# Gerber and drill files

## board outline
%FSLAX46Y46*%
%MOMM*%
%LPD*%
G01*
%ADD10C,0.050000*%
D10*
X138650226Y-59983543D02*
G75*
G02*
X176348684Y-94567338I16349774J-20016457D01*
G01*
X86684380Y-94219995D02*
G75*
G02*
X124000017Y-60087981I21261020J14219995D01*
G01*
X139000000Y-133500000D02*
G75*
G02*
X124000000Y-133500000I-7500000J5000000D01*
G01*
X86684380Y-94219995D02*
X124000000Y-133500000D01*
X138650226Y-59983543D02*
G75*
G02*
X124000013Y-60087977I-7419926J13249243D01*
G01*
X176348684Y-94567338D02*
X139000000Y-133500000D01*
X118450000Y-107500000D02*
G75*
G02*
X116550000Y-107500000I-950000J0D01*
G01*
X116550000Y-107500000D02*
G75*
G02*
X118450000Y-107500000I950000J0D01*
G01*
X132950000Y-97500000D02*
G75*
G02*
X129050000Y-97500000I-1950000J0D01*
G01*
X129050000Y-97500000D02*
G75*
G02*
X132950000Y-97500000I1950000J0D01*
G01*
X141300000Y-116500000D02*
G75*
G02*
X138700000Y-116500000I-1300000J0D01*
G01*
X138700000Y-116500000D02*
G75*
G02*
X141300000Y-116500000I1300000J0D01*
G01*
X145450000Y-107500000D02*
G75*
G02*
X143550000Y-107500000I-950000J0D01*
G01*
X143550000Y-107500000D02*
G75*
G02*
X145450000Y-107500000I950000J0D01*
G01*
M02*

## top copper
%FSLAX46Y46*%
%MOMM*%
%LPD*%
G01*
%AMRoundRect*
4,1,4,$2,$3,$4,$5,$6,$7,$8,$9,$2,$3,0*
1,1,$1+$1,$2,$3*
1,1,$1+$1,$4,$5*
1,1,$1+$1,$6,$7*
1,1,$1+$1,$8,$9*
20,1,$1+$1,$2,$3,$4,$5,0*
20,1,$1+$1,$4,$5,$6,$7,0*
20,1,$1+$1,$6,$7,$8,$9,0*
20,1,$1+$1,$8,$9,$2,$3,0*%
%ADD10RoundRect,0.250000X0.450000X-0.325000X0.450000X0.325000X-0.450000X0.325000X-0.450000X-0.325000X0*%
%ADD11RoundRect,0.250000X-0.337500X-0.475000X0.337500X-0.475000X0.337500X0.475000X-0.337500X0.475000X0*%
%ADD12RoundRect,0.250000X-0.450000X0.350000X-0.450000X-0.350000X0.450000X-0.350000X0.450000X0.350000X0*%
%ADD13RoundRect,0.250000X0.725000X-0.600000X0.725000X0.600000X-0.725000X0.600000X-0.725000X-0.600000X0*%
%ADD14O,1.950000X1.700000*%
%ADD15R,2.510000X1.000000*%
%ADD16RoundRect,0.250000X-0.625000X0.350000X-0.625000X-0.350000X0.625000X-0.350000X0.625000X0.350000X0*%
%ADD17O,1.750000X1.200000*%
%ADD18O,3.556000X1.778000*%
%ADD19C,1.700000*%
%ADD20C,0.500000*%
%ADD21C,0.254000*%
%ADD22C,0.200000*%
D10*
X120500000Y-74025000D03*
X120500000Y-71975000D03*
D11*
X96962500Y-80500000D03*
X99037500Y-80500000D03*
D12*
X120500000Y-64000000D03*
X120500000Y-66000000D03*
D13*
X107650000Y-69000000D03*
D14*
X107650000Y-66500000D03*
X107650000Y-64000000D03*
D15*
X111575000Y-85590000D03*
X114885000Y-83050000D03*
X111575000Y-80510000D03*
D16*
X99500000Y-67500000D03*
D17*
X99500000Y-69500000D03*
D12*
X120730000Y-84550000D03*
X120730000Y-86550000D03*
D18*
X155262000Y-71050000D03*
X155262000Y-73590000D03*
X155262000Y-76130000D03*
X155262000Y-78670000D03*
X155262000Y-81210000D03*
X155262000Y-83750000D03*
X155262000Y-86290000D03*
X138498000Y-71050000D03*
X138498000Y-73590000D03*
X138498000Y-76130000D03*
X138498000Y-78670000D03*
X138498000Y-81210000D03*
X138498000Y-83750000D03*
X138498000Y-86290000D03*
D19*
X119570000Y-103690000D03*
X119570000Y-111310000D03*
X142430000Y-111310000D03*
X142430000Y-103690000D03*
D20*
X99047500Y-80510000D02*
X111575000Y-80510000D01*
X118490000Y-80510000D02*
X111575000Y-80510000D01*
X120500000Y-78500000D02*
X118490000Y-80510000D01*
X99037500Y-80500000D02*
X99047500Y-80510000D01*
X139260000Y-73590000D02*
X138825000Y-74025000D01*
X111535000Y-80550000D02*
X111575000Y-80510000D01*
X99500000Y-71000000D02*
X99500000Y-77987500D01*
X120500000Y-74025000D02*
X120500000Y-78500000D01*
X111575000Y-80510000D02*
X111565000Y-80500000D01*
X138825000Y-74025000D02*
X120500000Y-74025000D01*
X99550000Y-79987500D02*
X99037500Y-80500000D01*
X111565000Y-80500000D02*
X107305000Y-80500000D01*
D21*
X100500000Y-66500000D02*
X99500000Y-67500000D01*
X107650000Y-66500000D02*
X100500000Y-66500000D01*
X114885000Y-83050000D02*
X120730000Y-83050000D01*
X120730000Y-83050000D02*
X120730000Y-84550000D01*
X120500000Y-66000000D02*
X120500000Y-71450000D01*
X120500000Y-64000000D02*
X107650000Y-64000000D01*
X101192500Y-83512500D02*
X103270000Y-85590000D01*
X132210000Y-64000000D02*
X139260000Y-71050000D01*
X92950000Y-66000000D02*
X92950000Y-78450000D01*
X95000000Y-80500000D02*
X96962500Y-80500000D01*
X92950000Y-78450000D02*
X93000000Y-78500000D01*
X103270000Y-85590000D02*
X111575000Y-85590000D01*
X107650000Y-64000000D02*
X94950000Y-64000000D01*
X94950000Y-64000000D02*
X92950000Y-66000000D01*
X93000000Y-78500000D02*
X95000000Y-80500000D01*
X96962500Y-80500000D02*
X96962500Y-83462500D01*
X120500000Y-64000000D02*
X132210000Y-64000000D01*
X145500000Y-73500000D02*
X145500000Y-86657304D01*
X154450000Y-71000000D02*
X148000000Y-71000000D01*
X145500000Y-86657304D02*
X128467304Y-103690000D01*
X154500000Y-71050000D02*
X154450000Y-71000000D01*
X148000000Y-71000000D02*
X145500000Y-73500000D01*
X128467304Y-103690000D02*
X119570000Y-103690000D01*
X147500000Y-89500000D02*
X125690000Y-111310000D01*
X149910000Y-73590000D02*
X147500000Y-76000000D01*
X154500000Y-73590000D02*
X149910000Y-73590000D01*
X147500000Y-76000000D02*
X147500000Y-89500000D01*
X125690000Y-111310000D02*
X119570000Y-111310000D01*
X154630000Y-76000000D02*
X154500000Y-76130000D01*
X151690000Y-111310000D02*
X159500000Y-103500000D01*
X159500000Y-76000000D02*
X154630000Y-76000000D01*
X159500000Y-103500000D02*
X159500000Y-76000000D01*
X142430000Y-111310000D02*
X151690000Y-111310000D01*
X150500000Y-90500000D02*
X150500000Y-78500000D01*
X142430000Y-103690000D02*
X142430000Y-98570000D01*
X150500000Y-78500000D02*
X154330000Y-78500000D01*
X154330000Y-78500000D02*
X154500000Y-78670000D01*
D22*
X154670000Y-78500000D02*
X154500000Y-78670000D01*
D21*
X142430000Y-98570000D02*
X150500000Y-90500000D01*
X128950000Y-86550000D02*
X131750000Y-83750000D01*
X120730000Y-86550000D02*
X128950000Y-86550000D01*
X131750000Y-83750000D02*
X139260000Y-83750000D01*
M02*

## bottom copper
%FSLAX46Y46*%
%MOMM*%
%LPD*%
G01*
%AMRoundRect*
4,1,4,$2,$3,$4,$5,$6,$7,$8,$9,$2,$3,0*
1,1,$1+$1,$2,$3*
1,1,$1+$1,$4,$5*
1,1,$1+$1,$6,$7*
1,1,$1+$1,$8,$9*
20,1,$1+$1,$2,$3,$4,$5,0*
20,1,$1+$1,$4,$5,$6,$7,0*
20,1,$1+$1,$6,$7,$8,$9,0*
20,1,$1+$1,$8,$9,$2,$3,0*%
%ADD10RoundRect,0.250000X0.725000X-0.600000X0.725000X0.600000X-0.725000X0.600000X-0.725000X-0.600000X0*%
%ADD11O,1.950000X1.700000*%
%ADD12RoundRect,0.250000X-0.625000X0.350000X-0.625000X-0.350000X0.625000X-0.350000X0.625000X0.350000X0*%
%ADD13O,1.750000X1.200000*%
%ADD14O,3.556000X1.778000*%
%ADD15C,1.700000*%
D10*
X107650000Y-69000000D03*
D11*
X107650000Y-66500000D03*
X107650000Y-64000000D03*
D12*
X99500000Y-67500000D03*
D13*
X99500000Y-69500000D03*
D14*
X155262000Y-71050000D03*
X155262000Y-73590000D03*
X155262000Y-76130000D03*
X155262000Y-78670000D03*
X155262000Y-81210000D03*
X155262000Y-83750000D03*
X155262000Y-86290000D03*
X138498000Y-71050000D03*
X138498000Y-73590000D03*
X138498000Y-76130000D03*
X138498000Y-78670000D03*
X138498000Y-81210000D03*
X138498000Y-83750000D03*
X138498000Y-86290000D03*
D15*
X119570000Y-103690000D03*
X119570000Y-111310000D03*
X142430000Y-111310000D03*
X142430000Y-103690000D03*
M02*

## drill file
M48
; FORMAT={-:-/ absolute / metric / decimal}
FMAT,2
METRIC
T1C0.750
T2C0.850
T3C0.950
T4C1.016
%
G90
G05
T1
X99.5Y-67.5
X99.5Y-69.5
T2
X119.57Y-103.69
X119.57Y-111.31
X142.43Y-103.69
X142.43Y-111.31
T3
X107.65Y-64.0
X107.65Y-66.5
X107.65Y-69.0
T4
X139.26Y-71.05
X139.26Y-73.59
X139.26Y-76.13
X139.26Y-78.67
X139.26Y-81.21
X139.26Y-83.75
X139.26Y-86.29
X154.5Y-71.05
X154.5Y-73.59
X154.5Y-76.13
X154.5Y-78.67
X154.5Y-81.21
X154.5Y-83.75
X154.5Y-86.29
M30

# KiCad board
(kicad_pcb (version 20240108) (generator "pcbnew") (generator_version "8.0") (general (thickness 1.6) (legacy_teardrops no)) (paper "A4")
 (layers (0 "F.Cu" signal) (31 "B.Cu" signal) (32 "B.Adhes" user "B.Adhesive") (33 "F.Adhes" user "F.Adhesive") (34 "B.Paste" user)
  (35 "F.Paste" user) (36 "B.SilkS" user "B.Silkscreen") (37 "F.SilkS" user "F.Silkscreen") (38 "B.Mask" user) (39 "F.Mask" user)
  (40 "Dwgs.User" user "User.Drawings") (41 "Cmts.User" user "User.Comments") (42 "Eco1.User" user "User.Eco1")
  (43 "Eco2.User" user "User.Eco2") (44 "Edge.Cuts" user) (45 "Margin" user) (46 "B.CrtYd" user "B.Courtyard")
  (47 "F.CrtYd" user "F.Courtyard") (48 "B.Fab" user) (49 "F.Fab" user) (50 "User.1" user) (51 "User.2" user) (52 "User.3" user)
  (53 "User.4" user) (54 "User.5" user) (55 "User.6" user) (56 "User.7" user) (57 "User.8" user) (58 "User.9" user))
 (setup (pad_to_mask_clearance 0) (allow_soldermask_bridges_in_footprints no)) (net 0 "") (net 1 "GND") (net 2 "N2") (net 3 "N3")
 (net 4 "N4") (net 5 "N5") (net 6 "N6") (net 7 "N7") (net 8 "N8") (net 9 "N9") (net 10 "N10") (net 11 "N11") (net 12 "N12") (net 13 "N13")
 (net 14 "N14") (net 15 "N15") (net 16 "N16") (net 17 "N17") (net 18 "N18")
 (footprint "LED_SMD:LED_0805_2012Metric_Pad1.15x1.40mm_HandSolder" (layer "F.Cu") (at 120.5 73 90)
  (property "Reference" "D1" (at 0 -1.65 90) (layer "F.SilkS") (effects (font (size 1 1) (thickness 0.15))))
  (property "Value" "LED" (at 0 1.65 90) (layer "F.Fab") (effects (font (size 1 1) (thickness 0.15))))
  (pad "1" smd roundrect (at -1.025 0 90) (size 1.15 1.4) (layers "F.Cu" "F.Paste" "F.Mask") (roundrect_rratio 0.217391) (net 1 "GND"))
  (pad "2" smd roundrect (at 1.025 0 90) (size 1.15 1.4) (layers "F.Cu" "F.Paste" "F.Mask") (roundrect_rratio 0.217391) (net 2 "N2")))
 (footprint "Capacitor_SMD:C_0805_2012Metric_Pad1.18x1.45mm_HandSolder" (layer "F.Cu") (at 98 80.5)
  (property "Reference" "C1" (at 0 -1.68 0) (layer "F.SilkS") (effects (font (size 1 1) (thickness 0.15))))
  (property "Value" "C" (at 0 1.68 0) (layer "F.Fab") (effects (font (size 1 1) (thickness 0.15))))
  (pad "1" smd roundrect (at -1.0375 0) (size 1.175 1.45) (layers "F.Cu" "F.Paste" "F.Mask") (roundrect_rratio 0.212766) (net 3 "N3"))
  (pad "2" smd roundrect (at 1.0375 0) (size 1.175 1.45) (layers "F.Cu" "F.Paste" "F.Mask") (roundrect_rratio 0.212766) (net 1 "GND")))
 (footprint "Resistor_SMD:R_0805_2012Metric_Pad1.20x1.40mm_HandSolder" (layer "F.Cu") (at 120.5 65 -90)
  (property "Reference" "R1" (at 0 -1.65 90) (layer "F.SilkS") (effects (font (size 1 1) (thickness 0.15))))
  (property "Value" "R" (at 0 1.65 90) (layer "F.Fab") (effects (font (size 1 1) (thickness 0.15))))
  (pad "1" smd roundrect (at -1 0 270) (size 1.2 1.4) (layers "F.Cu" "F.Paste" "F.Mask") (roundrect_rratio 0.208333) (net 3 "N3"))
  (pad "2" smd roundrect (at 1 0 270) (size 1.2 1.4) (layers "F.Cu" "F.Paste" "F.Mask") (roundrect_rratio 0.208333) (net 2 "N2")))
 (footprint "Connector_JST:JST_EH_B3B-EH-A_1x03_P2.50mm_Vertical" (layer "F.Cu") (at 107.65 69 90)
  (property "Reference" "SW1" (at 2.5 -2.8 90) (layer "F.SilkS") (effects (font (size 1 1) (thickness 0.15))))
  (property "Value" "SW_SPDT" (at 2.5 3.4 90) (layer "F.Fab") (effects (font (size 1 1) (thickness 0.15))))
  (pad "1" thru_hole roundrect (at 0 0 90) (size 1.7 1.95) (drill 0.95) (layers "*.Cu" "*.Mask") (remove_unused_layers no)
   (roundrect_rratio 0.147059) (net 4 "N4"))
  (pad "2" thru_hole oval (at 2.5 0 90) (size 1.7 1.95) (drill 0.95) (layers "*.Cu" "*.Mask") (remove_unused_layers no) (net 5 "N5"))
  (pad "3" thru_hole oval (at 5 0 90) (size 1.7 1.95) (drill 0.95) (layers "*.Cu" "*.Mask") (remove_unused_layers no) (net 3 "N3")))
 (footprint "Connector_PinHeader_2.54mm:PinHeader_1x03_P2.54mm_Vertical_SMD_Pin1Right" (layer "F.Cu") (at 113.23 83.05 180)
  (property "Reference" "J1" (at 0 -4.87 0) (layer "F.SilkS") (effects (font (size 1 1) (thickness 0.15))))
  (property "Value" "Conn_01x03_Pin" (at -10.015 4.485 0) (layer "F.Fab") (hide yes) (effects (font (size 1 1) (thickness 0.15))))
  (pad "1" smd rect (at 1.655 -2.54 180) (size 2.51 1) (layers "F.Cu" "F.Paste" "F.Mask") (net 3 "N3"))
  (pad "2" smd rect (at -1.655 0 180) (size 2.51 1) (layers "F.Cu" "F.Paste" "F.Mask") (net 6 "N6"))
  (pad "3" smd rect (at 1.655 2.54 180) (size 2.51 1) (layers "F.Cu" "F.Paste" "F.Mask") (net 1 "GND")))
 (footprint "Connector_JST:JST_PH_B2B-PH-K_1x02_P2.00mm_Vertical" (layer "F.Cu") (at 99.5 67.5 -90)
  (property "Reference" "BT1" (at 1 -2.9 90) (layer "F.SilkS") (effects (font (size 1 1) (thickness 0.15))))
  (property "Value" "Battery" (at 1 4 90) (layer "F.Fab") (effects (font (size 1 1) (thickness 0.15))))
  (pad "1" thru_hole roundrect (at 0 0 270) (size 1.2 1.75) (drill 0.75) (layers "*.Cu" "*.Mask") (remove_unused_layers no)
   (roundrect_rratio 0.208333) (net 5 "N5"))
  (pad "2" thru_hole oval (at 2 0 270) (size 1.2 1.75) (drill 0.75) (layers "*.Cu" "*.Mask") (remove_unused_layers no) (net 1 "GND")))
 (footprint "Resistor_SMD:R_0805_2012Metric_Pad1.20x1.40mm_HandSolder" (layer "F.Cu") (at 120.73 85.55 -90)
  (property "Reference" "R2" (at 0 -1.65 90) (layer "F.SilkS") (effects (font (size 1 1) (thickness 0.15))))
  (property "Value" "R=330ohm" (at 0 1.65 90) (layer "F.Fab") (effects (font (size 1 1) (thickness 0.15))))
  (pad "1" smd roundrect (at -1 0 270) (size 1.2 1.4) (layers "F.Cu" "F.Paste" "F.Mask") (roundrect_rratio 0.208333) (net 6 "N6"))
  (pad "2" smd roundrect (at 1 0 270) (size 1.2 1.4) (layers "F.Cu" "F.Paste" "F.Mask") (roundrect_rratio 0.208333) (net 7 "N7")))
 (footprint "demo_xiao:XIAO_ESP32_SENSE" (layer "B.Cu") (at 146.88 78.67 180)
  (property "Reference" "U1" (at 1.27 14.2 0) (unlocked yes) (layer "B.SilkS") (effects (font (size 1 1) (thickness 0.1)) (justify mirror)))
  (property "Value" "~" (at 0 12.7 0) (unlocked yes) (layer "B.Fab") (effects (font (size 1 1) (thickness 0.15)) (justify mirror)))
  (pad "1" thru_hole oval (at -7.62 7.62 180) (size 3.556 1.778) (drill 1.016 (offset -0.762 0)) (layers "*.Cu" "*.Mask")
   (remove_unused_layers no) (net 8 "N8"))
  (pad "2" thru_hole oval (at -7.62 5.08 180) (size 3.556 1.778) (drill 1.016 (offset -0.762 0)) (layers "*.Cu" "*.Mask")
   (remove_unused_layers no) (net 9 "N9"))
  (pad "3" thru_hole oval (at -7.62 2.54 180) (size 3.556 1.778) (drill 1.016 (offset -0.762 0)) (layers "*.Cu" "*.Mask")
   (remove_unused_layers no) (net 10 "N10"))
  (pad "4" thru_hole oval (at -7.62 0 180) (size 3.556 1.778) (drill 1.016 (offset -0.762 0)) (layers "*.Cu" "*.Mask")
   (remove_unused_layers no) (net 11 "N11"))
  (pad "5" thru_hole oval (at -7.62 -2.54 180) (size 3.556 1.778) (drill 1.016 (offset -0.762 0)) (layers "*.Cu" "*.Mask")
   (remove_unused_layers no) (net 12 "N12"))
  (pad "6" thru_hole oval (at -7.62 -5.08 180) (size 3.556 1.778) (drill 1.016 (offset -0.762 0)) (layers "*.Cu" "*.Mask")
   (remove_unused_layers no) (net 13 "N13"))
  (pad "7" thru_hole oval (at -7.62 -7.62 180) (size 3.556 1.778) (drill 1.016 (offset -0.762 0)) (layers "*.Cu" "*.Mask")
   (remove_unused_layers no) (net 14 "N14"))
  (pad "8" thru_hole oval (at 7.62 7.62 180) (size 3.556 1.778) (drill 1.016 (offset 0.762 0)) (layers "*.Cu" "*.Mask")
   (remove_unused_layers no) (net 3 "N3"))
  (pad "9" thru_hole oval (at 7.62 5.08 180) (size 3.556 1.778) (drill 1.016 (offset 0.762 0)) (layers "*.Cu" "*.Mask")
   (remove_unused_layers no) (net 1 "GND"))
  (pad "10" thru_hole oval (at 7.62 2.54 180) (size 3.556 1.778) (drill 1.016 (offset 0.762 0)) (layers "*.Cu" "*.Mask")
   (remove_unused_layers no) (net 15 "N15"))
  (pad "11" thru_hole oval (at 7.62 0 180) (size 3.556 1.778) (drill 1.016 (offset 0.762 0)) (layers "*.Cu" "*.Mask")
   (remove_unused_layers no) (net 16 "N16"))
  (pad "12" thru_hole oval (at 7.62 -2.54 180) (size 3.556 1.778) (drill 1.016 (offset 0.762 0)) (layers "*.Cu" "*.Mask")
   (remove_unused_layers no) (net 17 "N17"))
  (pad "13" thru_hole oval (at 7.62 -5.08 180) (size 3.556 1.778) (drill 1.016 (offset 0.762 0)) (layers "*.Cu" "*.Mask")
   (remove_unused_layers no) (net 7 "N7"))
  (pad "14" thru_hole oval (at 7.62 -7.62 180) (size 3.556 1.778) (drill 1.016 (offset 0.762 0)) (layers "*.Cu" "*.Mask")
   (remove_unused_layers no) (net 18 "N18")))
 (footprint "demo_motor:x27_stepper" (layer "B.Cu") (at 128.46 117.66 180)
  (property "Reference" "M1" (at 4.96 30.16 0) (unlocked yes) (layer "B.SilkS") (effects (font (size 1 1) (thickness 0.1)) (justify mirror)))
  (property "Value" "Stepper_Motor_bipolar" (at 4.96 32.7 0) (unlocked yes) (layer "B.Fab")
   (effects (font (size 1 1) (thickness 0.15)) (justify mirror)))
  (fp_circle (center 10.96 10.16) (end 11.91 10.16) (stroke (width 0.05) (type default)) (fill none) (layer "Edge.Cuts"))
  (fp_circle (center -2.54 20.16) (end -0.59 20.16) (stroke (width 0.05) (type default)) (fill none) (layer "Edge.Cuts"))
  (fp_circle (center -11.54 1.16) (end -10.24 1.16) (stroke (width 0.05) (type default)) (fill none) (layer "Edge.Cuts"))
  (fp_circle (center -16.04 10.16) (end -15.09 10.16) (stroke (width 0.05) (type default)) (fill none) (layer "Edge.Cuts"))
  (pad "1" thru_hole circle (at 8.89 13.97 180) (size 1.7 1.7) (drill 0.85) (layers "*.Cu" "*.Mask") (remove_unused_layers no) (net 8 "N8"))
  (pad "2" thru_hole circle (at 8.89 6.35 180) (size 1.7 1.7) (drill 0.85) (layers "*.Cu" "*.Mask") (remove_unused_layers no) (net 9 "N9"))
  (pad "3" thru_hole circle (at -13.97 6.35 180) (size 1.7 1.7) (drill 0.85) (layers "*.Cu" "*.Mask") (remove_unused_layers no)
   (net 10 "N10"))
  (pad "4" thru_hole circle (at -13.97 13.97 180) (size 1.7 1.7) (drill 0.85) (layers "*.Cu" "*.Mask") (remove_unused_layers no)
   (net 11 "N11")))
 (gr_arc (start 138.650226 59.983543) (mid 172.471605 60.954878) (end 176.348684 94.567338) (stroke (width 0.05) (type default))
  (layer "Edge.Cuts"))
 (gr_arc (start 86.68438 94.219995) (mid 90.681985 61.126378) (end 124 60.088002) (stroke (width 0.05) (type default)) (layer "Edge.Cuts"))
 (gr_arc (start 139 133.5) (mid 131.5 137.513878) (end 124 133.5) (stroke (width 0.05) (type default)) (layer "Edge.Cuts"))
 (gr_line (start 86.68438 94.219995) (end 124 133.5) (stroke (width 0.05) (type default)) (layer "Edge.Cuts"))
 (gr_arc (start 138.650226 59.983543) (mid 131.338543 61.919371) (end 124 60.088002) (stroke (width 0.05) (type default))
  (layer "Edge.Cuts"))
 (gr_line (start 176.348684 94.567338) (end 139 133.5) (stroke (width 0.05) (type default)) (layer "Edge.Cuts"))
 (segment (start 99.0475 80.51) (end 111.575 80.51) (width 0.5) (layer "F.Cu") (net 1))
 (segment (start 118.49 80.51) (end 111.575 80.51) (width 0.5) (layer "F.Cu") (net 1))
 (segment (start 120.5 78.5) (end 118.49 80.51) (width 0.5) (layer "F.Cu") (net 1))
 (segment (start 99.0375 80.5) (end 99.0475 80.51) (width 0.5) (layer "F.Cu") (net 1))
 (segment (start 139.26 73.59) (end 138.825 74.025) (width 0.5) (layer "F.Cu") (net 1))
 (segment (start 111.535 80.55) (end 111.575 80.51) (width 0.5) (layer "F.Cu") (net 1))
 (segment (start 99.5 71) (end 99.5 77.9875) (width 0.5) (layer "F.Cu") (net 1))
 (segment (start 120.5 74.025) (end 120.5 78.5) (width 0.5) (layer "F.Cu") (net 1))
 (segment (start 111.575 80.51) (end 111.565 80.5) (width 0.5) (layer "F.Cu") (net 1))
 (segment (start 138.825 74.025) (end 120.5 74.025) (width 0.5) (layer "F.Cu") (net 1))
 (segment (start 99.55 79.9875) (end 99.0375 80.5) (width 0.5) (layer "F.Cu") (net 1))
 (segment (start 111.565 80.5) (end 107.305 80.5) (width 0.5) (layer "F.Cu") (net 1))
 (segment (start 100.5 66.5) (end 99.5 67.5) (width 0.254) (layer "F.Cu") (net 5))
 (segment (start 107.65 66.5) (end 100.5 66.5) (width 0.254) (layer "F.Cu") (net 5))
 (segment (start 114.885 83.05) (end 120.73 83.05) (width 0.254) (layer "F.Cu") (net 6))
 (segment (start 120.73 83.05) (end 120.73 84.55) (width 0.254) (layer "F.Cu") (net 6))
 (segment (start 120.5 66) (end 120.5 71.45) (width 0.254) (layer "F.Cu") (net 2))
 (segment (start 120.5 64) (end 107.65 64) (width 0.254) (layer "F.Cu") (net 3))
 (segment (start 101.1925 83.5125) (end 103.27 85.59) (width 0.254) (layer "F.Cu") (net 3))
 (segment (start 132.21 64) (end 139.26 71.05) (width 0.254) (layer "F.Cu") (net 3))
 (segment (start 92.95 66) (end 92.95 78.45) (width 0.254) (layer "F.Cu") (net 3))
 (segment (start 95 80.5) (end 96.9625 80.5) (width 0.254) (layer "F.Cu") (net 3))
 (segment (start 92.95 78.45) (end 93 78.5) (width 0.254) (layer "F.Cu") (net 3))
 (segment (start 103.27 85.59) (end 111.575 85.59) (width 0.254) (layer "F.Cu") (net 3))
 (segment (start 107.65 64) (end 94.95 64) (width 0.254) (layer "F.Cu") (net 3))
 (segment (start 94.95 64) (end 92.95 66) (width 0.254) (layer "F.Cu") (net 3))
 (segment (start 93 78.5) (end 95 80.5) (width 0.254) (layer "F.Cu") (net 3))
 (segment (start 96.9625 80.5) (end 96.9625 83.4625) (width 0.254) (layer "F.Cu") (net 3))
 (segment (start 120.5 64) (end 132.21 64) (width 0.254) (layer "F.Cu") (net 3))
 (segment (start 145.5 73.5) (end 145.5 86.657304) (width 0.254) (layer "F.Cu") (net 8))
 (segment (start 154.45 71) (end 148 71) (width 0.254) (layer "F.Cu") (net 8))
 (segment (start 145.5 86.657304) (end 128.467304 103.69) (width 0.254) (layer "F.Cu") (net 8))
 (segment (start 154.5 71.05) (end 154.45 71) (width 0.254) (layer "F.Cu") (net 8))
 (segment (start 148 71) (end 145.5 73.5) (width 0.254) (layer "F.Cu") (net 8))
 (segment (start 128.467304 103.69) (end 119.57 103.69) (width 0.254) (layer "F.Cu") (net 8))
 (segment (start 147.5 89.5) (end 125.69 111.31) (width 0.254) (layer "F.Cu") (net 9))
 (segment (start 149.91 73.59) (end 147.5 76) (width 0.254) (layer "F.Cu") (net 9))
 (segment (start 154.5 73.59) (end 149.91 73.59) (width 0.254) (layer "F.Cu") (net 9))
 (segment (start 147.5 76) (end 147.5 89.5) (width 0.254) (layer "F.Cu") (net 9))
 (segment (start 125.69 111.31) (end 119.57 111.31) (width 0.254) (layer "F.Cu") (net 9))
 (segment (start 154.63 76) (end 154.5 76.13) (width 0.254) (layer "F.Cu") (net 10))
 (segment (start 151.69 111.31) (end 159.5 103.5) (width 0.254) (layer "F.Cu") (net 10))
 (segment (start 159.5 76) (end 154.63 76) (width 0.254) (layer "F.Cu") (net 10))
 (segment (start 159.5 103.5) (end 159.5 76) (width 0.254) (layer "F.Cu") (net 10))
 (segment (start 142.43 111.31) (end 151.69 111.31) (width 0.254) (layer "F.Cu") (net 10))
 (segment (start 150.5 90.5) (end 150.5 78.5) (width 0.254) (layer "F.Cu") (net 11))
 (segment (start 142.43 103.69) (end 142.43 98.57) (width 0.254) (layer "F.Cu") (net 11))
 (segment (start 150.5 78.5) (end 154.33 78.5) (width 0.254) (layer "F.Cu") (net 11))
 (segment (start 154.33 78.5) (end 154.5 78.67) (width 0.254) (layer "F.Cu") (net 11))
 (segment (start 154.67 78.5) (end 154.5 78.67) (width 0.2) (layer "F.Cu") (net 11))
 (segment (start 142.43 98.57) (end 150.5 90.5) (width 0.254) (layer "F.Cu") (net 11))
 (segment (start 128.95 86.55) (end 131.75 83.75) (width 0.254) (layer "F.Cu") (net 7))
 (segment (start 120.73 86.55) (end 128.95 86.55) (width 0.254) (layer "F.Cu") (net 7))
 (segment (start 131.75 83.75) (end 139.26 83.75) (width 0.254) (layer "F.Cu") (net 7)))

